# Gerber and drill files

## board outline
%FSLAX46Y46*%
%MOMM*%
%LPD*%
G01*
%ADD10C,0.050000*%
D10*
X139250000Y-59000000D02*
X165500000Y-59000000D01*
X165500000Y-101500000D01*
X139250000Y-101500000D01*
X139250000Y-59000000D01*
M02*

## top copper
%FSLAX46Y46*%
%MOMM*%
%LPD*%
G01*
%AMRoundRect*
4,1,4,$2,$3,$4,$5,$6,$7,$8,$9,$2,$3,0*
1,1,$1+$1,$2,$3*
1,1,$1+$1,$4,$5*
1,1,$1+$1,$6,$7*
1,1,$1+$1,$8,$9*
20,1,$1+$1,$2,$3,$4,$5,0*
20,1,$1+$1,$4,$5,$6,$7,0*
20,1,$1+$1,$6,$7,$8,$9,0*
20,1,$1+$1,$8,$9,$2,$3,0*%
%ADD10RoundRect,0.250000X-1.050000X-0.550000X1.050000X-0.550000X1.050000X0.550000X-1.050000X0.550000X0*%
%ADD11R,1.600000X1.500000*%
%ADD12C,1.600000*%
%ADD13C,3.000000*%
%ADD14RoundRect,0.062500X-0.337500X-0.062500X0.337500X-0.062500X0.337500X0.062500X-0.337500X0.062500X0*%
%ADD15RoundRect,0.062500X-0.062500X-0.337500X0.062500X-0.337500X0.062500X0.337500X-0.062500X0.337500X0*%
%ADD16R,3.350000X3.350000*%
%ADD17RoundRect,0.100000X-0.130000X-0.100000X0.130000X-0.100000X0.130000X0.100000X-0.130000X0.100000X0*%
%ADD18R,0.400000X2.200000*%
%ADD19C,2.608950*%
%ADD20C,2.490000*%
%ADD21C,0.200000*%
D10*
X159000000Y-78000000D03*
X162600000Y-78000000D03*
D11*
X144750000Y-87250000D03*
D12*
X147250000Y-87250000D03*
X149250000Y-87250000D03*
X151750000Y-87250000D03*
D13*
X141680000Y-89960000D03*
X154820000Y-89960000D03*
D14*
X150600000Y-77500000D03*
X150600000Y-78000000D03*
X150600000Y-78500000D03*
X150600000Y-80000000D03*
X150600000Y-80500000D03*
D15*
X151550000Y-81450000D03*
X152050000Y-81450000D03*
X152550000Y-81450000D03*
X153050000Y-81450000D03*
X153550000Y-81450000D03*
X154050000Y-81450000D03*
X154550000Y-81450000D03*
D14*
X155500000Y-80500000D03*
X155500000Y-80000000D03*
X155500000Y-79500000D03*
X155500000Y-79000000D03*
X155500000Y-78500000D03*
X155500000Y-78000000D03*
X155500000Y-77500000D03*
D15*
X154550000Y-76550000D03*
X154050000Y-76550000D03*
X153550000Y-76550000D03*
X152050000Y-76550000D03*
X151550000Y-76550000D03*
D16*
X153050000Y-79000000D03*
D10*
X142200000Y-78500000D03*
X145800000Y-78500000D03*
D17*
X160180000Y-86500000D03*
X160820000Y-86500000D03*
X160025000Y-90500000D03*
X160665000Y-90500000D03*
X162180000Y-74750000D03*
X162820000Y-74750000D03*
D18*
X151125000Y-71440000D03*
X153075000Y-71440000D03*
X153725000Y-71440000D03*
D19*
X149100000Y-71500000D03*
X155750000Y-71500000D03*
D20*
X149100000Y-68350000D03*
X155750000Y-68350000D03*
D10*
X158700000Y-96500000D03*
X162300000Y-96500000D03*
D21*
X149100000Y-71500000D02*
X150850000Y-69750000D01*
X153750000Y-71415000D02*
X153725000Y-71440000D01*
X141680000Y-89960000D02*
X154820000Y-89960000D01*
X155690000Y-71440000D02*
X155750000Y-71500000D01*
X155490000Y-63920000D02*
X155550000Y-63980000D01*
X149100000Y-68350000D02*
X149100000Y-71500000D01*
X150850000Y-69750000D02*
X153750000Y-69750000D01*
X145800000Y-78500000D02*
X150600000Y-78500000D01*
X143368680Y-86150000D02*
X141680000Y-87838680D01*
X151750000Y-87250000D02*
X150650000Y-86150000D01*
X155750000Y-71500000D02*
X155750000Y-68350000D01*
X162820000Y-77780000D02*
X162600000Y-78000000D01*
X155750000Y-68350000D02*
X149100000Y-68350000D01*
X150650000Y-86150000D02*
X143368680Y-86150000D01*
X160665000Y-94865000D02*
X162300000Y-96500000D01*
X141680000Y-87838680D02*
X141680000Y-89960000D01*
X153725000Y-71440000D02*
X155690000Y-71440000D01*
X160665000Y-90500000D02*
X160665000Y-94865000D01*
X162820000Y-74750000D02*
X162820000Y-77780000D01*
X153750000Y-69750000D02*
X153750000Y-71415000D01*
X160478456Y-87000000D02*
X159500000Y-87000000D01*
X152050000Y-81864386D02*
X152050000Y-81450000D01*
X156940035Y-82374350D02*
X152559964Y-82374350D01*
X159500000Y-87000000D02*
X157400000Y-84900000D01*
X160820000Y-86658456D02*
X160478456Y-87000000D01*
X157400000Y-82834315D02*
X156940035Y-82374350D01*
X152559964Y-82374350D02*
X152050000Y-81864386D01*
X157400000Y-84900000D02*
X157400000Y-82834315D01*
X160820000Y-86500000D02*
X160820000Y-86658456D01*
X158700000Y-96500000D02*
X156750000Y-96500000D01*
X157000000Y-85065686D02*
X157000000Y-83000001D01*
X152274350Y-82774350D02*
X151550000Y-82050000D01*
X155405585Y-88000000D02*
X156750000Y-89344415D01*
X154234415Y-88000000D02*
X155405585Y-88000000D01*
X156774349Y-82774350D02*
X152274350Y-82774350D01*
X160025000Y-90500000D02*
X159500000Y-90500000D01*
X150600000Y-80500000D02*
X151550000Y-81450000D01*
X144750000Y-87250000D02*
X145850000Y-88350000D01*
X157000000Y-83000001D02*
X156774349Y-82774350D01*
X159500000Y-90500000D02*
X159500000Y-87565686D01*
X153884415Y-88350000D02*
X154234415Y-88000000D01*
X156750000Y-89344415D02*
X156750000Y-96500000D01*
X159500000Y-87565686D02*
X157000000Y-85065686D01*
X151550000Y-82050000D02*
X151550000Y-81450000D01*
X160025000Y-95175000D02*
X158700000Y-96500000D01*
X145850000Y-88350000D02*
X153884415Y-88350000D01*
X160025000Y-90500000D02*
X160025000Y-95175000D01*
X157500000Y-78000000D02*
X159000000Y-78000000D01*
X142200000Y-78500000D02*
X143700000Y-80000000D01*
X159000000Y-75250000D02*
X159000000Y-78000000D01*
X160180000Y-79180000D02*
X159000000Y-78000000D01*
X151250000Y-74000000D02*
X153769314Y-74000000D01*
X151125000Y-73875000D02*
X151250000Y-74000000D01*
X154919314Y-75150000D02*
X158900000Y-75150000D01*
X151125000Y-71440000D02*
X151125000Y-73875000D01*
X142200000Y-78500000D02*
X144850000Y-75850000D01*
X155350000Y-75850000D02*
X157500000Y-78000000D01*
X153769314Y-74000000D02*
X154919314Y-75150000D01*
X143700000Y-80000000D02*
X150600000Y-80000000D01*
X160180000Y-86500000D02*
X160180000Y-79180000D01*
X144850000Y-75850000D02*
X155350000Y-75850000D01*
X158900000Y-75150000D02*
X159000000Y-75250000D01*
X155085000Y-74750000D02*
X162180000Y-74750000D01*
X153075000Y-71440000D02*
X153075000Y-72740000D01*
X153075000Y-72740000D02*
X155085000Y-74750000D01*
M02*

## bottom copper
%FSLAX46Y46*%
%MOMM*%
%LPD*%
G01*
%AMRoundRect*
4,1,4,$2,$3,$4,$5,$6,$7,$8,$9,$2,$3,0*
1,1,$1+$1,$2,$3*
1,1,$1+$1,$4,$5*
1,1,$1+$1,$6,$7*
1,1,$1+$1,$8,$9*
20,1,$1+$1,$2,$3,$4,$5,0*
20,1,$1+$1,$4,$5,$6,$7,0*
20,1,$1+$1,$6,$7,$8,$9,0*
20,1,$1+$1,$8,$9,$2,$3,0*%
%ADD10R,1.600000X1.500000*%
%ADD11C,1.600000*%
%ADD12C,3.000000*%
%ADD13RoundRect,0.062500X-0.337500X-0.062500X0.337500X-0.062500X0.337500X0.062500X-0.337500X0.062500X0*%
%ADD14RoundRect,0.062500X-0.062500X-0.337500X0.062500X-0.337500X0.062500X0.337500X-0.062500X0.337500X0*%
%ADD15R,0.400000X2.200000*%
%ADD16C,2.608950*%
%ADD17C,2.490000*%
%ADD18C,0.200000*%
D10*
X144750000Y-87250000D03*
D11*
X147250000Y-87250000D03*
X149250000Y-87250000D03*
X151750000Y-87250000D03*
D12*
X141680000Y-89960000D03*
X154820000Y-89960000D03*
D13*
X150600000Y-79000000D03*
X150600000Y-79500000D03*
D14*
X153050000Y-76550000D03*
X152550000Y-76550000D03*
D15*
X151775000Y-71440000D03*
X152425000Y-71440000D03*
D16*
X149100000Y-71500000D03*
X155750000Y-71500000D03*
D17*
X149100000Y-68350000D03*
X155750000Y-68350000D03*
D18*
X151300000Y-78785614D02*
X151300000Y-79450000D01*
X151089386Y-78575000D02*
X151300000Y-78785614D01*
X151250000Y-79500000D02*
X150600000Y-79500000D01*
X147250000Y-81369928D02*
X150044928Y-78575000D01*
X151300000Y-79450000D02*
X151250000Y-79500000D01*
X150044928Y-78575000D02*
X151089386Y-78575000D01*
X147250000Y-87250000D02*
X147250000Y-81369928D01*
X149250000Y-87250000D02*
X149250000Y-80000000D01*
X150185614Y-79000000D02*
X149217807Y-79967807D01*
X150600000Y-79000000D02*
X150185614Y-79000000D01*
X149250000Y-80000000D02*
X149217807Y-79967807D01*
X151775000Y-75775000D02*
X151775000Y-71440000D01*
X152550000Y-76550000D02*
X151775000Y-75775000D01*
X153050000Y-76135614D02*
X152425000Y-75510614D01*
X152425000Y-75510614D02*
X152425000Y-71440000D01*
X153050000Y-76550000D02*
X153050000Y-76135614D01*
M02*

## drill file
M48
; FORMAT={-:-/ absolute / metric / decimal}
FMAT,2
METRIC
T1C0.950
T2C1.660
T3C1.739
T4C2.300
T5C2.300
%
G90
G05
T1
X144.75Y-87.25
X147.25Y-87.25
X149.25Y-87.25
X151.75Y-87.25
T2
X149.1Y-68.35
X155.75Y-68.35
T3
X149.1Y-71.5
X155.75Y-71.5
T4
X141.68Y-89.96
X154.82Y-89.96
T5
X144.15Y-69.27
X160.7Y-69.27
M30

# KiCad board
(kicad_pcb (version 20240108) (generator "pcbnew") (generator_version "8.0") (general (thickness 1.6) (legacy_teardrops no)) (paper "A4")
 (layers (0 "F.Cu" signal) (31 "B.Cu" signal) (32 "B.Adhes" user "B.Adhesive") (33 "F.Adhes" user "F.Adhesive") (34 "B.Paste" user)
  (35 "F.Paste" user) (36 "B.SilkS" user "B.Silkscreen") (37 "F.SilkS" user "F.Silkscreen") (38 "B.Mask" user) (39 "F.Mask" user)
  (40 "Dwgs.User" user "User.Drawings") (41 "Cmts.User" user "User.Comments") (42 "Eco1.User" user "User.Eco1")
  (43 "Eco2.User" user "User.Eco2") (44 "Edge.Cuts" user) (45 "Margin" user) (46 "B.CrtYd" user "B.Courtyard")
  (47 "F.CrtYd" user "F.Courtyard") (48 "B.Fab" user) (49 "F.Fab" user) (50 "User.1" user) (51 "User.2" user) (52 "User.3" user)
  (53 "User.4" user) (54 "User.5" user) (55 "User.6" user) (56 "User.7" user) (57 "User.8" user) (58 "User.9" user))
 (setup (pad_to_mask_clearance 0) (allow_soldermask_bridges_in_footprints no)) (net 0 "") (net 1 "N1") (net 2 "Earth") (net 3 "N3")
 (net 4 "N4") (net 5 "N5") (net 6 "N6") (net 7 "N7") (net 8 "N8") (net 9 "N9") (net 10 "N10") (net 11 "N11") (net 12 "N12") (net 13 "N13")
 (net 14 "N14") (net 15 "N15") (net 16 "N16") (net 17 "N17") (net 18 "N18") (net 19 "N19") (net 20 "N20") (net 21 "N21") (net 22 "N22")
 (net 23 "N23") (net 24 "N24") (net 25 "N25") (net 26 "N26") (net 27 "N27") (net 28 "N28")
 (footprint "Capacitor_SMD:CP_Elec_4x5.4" (layer "F.Cu") (at 160.8 78)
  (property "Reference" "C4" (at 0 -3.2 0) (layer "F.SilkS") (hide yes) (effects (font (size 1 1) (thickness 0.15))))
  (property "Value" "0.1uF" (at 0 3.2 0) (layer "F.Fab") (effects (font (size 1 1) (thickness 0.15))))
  (pad "1" smd roundrect (at -1.8 0) (size 2.6 1.6) (layers "F.Cu" "F.Paste" "F.Mask") (roundrect_rratio 0.15625) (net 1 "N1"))
  (pad "2" smd roundrect (at 1.8 0) (size 2.6 1.6) (layers "F.Cu" "F.Paste" "F.Mask") (roundrect_rratio 0.15625) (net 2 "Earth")))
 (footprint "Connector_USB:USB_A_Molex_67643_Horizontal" (layer "F.Cu") (at 144.75 87.25)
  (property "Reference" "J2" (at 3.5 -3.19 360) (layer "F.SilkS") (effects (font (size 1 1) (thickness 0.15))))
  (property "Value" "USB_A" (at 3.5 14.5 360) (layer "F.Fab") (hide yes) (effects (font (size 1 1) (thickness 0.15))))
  (pad "1" thru_hole rect (at 0 0) (size 1.6 1.5) (drill 0.95) (layers "*.Cu" "*.Mask") (remove_unused_layers no) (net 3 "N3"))
  (pad "2" thru_hole circle (at 2.5 0) (size 1.6 1.6) (drill 0.95) (layers "*.Cu" "*.Mask") (remove_unused_layers no) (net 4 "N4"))
  (pad "3" thru_hole circle (at 4.5 0) (size 1.6 1.6) (drill 0.95) (layers "*.Cu" "*.Mask") (remove_unused_layers no) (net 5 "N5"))
  (pad "4" thru_hole circle (at 7 0) (size 1.6 1.6) (drill 0.95) (layers "*.Cu" "*.Mask") (remove_unused_layers no) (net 2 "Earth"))
  (pad "5" thru_hole circle (at -3.07 2.71) (size 3 3) (drill 2.3) (layers "*.Cu" "*.Mask") (remove_unused_layers no) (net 2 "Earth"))
  (pad "5" thru_hole circle (at 10.07 2.71) (size 3 3) (drill 2.3) (layers "*.Cu" "*.Mask") (remove_unused_layers no) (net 2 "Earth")))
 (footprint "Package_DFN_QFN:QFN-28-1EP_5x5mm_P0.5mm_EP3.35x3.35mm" (layer "F.Cu") (at 153.05 79)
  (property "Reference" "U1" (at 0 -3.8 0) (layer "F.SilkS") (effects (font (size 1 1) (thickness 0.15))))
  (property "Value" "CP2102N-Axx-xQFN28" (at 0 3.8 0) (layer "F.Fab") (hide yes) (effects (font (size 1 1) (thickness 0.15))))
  (pad "" smd roundrect (at -1.12 -1.12) (size 0.9 0.9) (layers "F.Paste") (roundrect_rratio 0.25))
  (pad "" smd roundrect (at -1.12 0) (size 0.9 0.9) (layers "F.Paste") (roundrect_rratio 0.25))
  (pad "" smd roundrect (at -1.12 1.12) (size 0.9 0.9) (layers "F.Paste") (roundrect_rratio 0.25))
  (pad "" smd roundrect (at 0 -1.12) (size 0.9 0.9) (layers "F.Paste") (roundrect_rratio 0.25))
  (pad "" smd roundrect (at 0 0) (size 0.9 0.9) (layers "F.Paste") (roundrect_rratio 0.25))
  (pad "" smd roundrect (at 0 1.12) (size 0.9 0.9) (layers "F.Paste") (roundrect_rratio 0.25))
  (pad "" smd roundrect (at 1.12 -1.12) (size 0.9 0.9) (layers "F.Paste") (roundrect_rratio 0.25))
  (pad "" smd roundrect (at 1.12 0) (size 0.9 0.9) (layers "F.Paste") (roundrect_rratio 0.25))
  (pad "" smd roundrect (at 1.12 1.12) (size 0.9 0.9) (layers "F.Paste") (roundrect_rratio 0.25))
  (pad "1" smd roundrect (at -2.45 -1.5) (size 0.8 0.25) (layers "F.Cu" "F.Paste" "F.Mask") (roundrect_rratio 0.25) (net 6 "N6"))
  (pad "2" smd roundrect (at -2.45 -1) (size 0.8 0.25) (layers "F.Cu" "F.Paste" "F.Mask") (roundrect_rratio 0.25) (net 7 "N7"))
  (pad "3" smd roundrect (at -2.45 -0.5) (size 0.8 0.25) (layers "F.Cu" "F.Paste" "F.Mask") (roundrect_rratio 0.25) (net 2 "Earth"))
  (pad "4" smd roundrect (at -2.45 0) (size 0.8 0.25) (layers "B.Cu" "F.Paste" "F.Mask") (roundrect_rratio 0.25) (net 5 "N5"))
  (pad "5" smd roundrect (at -2.45 0.5) (size 0.8 0.25) (layers "B.Cu" "F.Paste" "F.Mask") (roundrect_rratio 0.25) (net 4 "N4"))
  (pad "6" smd roundrect (at -2.45 1) (size 0.8 0.25) (layers "F.Cu" "F.Paste" "F.Mask") (roundrect_rratio 0.25) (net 1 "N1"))
  (pad "7" smd roundrect (at -2.45 1.5) (size 0.8 0.25) (layers "F.Cu" "F.Paste" "F.Mask") (roundrect_rratio 0.25) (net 3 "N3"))
  (pad "8" smd roundrect (at -1.5 2.45) (size 0.25 0.8) (layers "F.Cu" "F.Paste" "F.Mask") (roundrect_rratio 0.25) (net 3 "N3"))
  (pad "9" smd roundrect (at -1 2.45) (size 0.25 0.8) (layers "F.Cu" "F.Paste" "F.Mask") (roundrect_rratio 0.25) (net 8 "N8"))
  (pad "10" smd roundrect (at -0.5 2.45) (size 0.25 0.8) (layers "F.Cu" "F.Paste" "F.Mask") (roundrect_rratio 0.25) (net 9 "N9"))
  (pad "11" smd roundrect (at 0 2.45) (size 0.25 0.8) (layers "F.Cu" "F.Paste" "F.Mask") (roundrect_rratio 0.25) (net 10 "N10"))
  (pad "12" smd roundrect (at 0.5 2.45) (size 0.25 0.8) (layers "F.Cu" "F.Paste" "F.Mask") (roundrect_rratio 0.25) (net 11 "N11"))
  (pad "13" smd roundrect (at 1 2.45) (size 0.25 0.8) (layers "F.Cu" "F.Paste" "F.Mask") (roundrect_rratio 0.25) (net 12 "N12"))
  (pad "14" smd roundrect (at 1.5 2.45) (size 0.25 0.8) (layers "F.Cu" "F.Paste" "F.Mask") (roundrect_rratio 0.25) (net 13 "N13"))
  (pad "15" smd roundrect (at 2.45 1.5) (size 0.8 0.25) (layers "F.Cu" "F.Paste" "F.Mask") (roundrect_rratio 0.25) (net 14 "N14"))
  (pad "16" smd roundrect (at 2.45 1) (size 0.8 0.25) (layers "F.Cu" "F.Paste" "F.Mask") (roundrect_rratio 0.25) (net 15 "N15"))
  (pad "17" smd roundrect (at 2.45 0.5) (size 0.8 0.25) (layers "F.Cu" "F.Paste" "F.Mask") (roundrect_rratio 0.25) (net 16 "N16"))
  (pad "18" smd roundrect (at 2.45 0) (size 0.8 0.25) (layers "F.Cu" "F.Paste" "F.Mask") (roundrect_rratio 0.25) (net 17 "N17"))
  (pad "19" smd roundrect (at 2.45 -0.5) (size 0.8 0.25) (layers "F.Cu" "F.Paste" "F.Mask") (roundrect_rratio 0.25) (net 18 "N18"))
  (pad "20" smd roundrect (at 2.45 -1) (size 0.8 0.25) (layers "F.Cu" "F.Paste" "F.Mask") (roundrect_rratio 0.25) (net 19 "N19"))
  (pad "21" smd roundrect (at 2.45 -1.5) (size 0.8 0.25) (layers "F.Cu" "F.Paste" "F.Mask") (roundrect_rratio 0.25) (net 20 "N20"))
  (pad "22" smd roundrect (at 1.5 -2.45) (size 0.25 0.8) (layers "F.Cu" "F.Paste" "F.Mask") (roundrect_rratio 0.25) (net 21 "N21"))
  (pad "23" smd roundrect (at 1 -2.45) (size 0.25 0.8) (layers "F.Cu" "F.Paste" "F.Mask") (roundrect_rratio 0.25) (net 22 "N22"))
  (pad "24" smd roundrect (at 0.5 -2.45) (size 0.25 0.8) (layers "F.Cu" "F.Paste" "F.Mask") (roundrect_rratio 0.25) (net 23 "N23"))
  (pad "25" smd roundrect (at 0 -2.45) (size 0.25 0.8) (layers "B.Cu" "F.Paste" "F.Mask") (roundrect_rratio 0.25) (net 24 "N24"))
  (pad "26" smd roundrect (at -0.5 -2.45) (size 0.25 0.8) (layers "B.Cu" "F.Paste" "F.Mask") (roundrect_rratio 0.25) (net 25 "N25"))
  (pad "27" smd roundrect (at -1 -2.45) (size 0.25 0.8) (layers "F.Cu" "F.Paste" "F.Mask") (roundrect_rratio 0.25) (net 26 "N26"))
  (pad "28" smd roundrect (at -1.5 -2.45) (size 0.25 0.8) (layers "F.Cu" "F.Paste" "F.Mask") (roundrect_rratio 0.25) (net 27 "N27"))
  (pad "29" smd rect (at 0 0) (size 3.35 3.35) (layers "F.Cu" "F.Mask") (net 2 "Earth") (zone_connect 2)))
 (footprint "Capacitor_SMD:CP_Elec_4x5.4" (layer "F.Cu") (at 144 78.5)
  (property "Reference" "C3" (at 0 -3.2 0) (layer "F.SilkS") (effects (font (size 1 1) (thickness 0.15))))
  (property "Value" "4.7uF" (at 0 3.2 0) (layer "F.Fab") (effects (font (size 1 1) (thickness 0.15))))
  (pad "1" smd roundrect (at -1.8 0) (size 2.6 1.6) (layers "F.Cu" "F.Paste" "F.Mask") (roundrect_rratio 0.15625) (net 1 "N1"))
  (pad "2" smd roundrect (at 1.8 0) (size 2.6 1.6) (layers "F.Cu" "F.Paste" "F.Mask") (roundrect_rratio 0.15625) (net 2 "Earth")))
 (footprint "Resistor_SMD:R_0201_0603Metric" (layer "F.Cu") (at 160.5 86.5)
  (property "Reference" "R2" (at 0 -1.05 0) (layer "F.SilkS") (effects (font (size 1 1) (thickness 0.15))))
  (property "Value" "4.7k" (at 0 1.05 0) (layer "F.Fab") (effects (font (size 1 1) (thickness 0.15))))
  (pad "" smd roundrect (at -0.345 0) (size 0.318 0.36) (layers "F.Paste") (roundrect_rratio 0.25))
  (pad "" smd roundrect (at 0.345 0) (size 0.318 0.36) (layers "F.Paste") (roundrect_rratio 0.25))
  (pad "1" smd roundrect (at -0.32 0) (size 0.46 0.4) (layers "F.Cu" "F.Mask") (roundrect_rratio 0.25) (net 1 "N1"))
  (pad "2" smd roundrect (at 0.32 0) (size 0.46 0.4) (layers "F.Cu" "F.Mask") (roundrect_rratio 0.25) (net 8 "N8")))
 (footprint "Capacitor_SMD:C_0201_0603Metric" (layer "F.Cu") (at 160.345 90.5)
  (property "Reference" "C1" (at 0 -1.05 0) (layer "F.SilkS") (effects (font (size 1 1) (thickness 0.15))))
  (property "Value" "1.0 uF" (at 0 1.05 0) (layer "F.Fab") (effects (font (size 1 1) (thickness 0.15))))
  (pad "" smd roundrect (at -0.345 0) (size 0.318 0.36) (layers "F.Paste") (roundrect_rratio 0.25))
  (pad "" smd roundrect (at 0.345 0) (size 0.318 0.36) (layers "F.Paste") (roundrect_rratio 0.25))
  (pad "1" smd roundrect (at -0.32 0) (size 0.46 0.4) (layers "F.Cu" "F.Mask") (roundrect_rratio 0.25) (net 3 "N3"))
  (pad "2" smd roundrect (at 0.32 0) (size 0.46 0.4) (layers "F.Cu" "F.Mask") (roundrect_rratio 0.25) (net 2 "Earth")))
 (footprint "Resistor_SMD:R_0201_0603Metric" (layer "F.Cu") (at 162.5 74.75)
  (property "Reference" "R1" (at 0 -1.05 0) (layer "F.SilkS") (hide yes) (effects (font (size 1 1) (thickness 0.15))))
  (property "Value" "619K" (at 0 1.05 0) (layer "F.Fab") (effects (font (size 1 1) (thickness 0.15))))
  (pad "" smd roundrect (at -0.345 0) (size 0.318 0.36) (layers "F.Paste") (roundrect_rratio 0.25))
  (pad "" smd roundrect (at 0.345 0) (size 0.318 0.36) (layers "F.Paste") (roundrect_rratio 0.25))
  (pad "1" smd roundrect (at -0.32 0) (size 0.46 0.4) (layers "F.Cu" "F.Mask") (roundrect_rratio 0.25) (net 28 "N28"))
  (pad "2" smd roundrect (at 0.32 0) (size 0.46 0.4) (layers "F.Cu" "F.Mask") (roundrect_rratio 0.25) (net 2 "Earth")))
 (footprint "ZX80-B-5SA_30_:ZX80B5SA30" (layer "F.Cu") (at 152.425 69.462)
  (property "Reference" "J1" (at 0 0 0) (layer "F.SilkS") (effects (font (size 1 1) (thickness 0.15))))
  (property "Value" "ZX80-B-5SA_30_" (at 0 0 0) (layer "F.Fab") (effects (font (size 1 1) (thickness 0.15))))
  (pad "" np_thru_hole circle (at -8.275 -0.192) (size 2.3 2.3) (drill 2.3) (layers "*.Cu" "*.Mask"))
  (pad "" np_thru_hole circle (at 8.275 -0.192) (size 2.3 2.3) (drill 2.3) (layers "*.Cu" "*.Mask"))
  (pad "1" smd rect (at -1.3 1.978 90) (size 2.2 0.4) (layers "F.Cu" "F.Paste" "F.Mask") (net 1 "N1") (solder_mask_margin 0.102))
  (pad "2" smd rect (at -0.65 1.978 90) (size 2.2 0.4) (layers "B.Cu" "F.Paste" "F.Mask") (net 25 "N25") (solder_mask_margin 0.102))
  (pad "3" smd rect (at 0 1.978 90) (size 2.2 0.4) (layers "B.Cu" "F.Paste" "F.Mask") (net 24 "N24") (solder_mask_margin 0.102))
  (pad "4" smd rect (at 0.65 1.978 90) (size 2.2 0.4) (layers "F.Cu" "F.Paste" "F.Mask") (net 28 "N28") (solder_mask_margin 0.102))
  (pad "5" smd rect (at 1.3 1.978 90) (size 2.2 0.4) (layers "F.Cu" "F.Paste" "F.Mask") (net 2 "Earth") (solder_mask_margin 0.102))
  (pad "6" thru_hole circle (at -3.325 2.038) (size 2.60895 2.60895) (drill 1.7393) (layers "*.Cu" "*.Mask") (remove_unused_layers no)
   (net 2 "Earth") (solder_mask_margin 0.102))
  (pad "7" thru_hole circle (at 3.325 2.038) (size 2.60895 2.60895) (drill 1.7393) (layers "*.Cu" "*.Mask") (remove_unused_layers no)
   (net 2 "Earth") (solder_mask_margin 0.102))
  (pad "8" thru_hole circle (at -3.325 -1.112) (size 2.49 2.49) (drill 1.66) (layers "*.Cu" "*.Mask") (remove_unused_layers no)
   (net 2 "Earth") (solder_mask_margin 0.102))
  (pad "9" thru_hole circle (at 3.325 -1.112) (size 2.49 2.49) (drill 1.66) (layers "*.Cu" "*.Mask") (remove_unused_layers no)
   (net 2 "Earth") (solder_mask_margin 0.102)))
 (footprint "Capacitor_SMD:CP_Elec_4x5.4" (layer "F.Cu") (at 160.5 96.5)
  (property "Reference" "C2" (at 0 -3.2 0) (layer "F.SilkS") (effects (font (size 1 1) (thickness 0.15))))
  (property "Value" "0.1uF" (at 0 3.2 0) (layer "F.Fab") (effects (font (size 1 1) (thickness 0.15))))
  (pad "1" smd roundrect (at -1.8 0) (size 2.6 1.6) (layers "F.Cu" "F.Paste" "F.Mask") (roundrect_rratio 0.15625) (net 3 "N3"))
  (pad "2" smd roundrect (at 1.8 0) (size 2.6 1.6) (layers "F.Cu" "F.Paste" "F.Mask") (roundrect_rratio 0.15625) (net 2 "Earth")))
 (gr_rect (start 139.25 59) (end 165.5 101.5) (stroke (width 0.05) (type default)) (fill none) (layer "Edge.Cuts"))
 (segment (start 149.1 71.5) (end 150.85 69.75) (width 0.2) (layer "F.Cu") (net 2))
 (segment (start 153.75 71.415) (end 153.725 71.44) (width 0.2) (layer "F.Cu") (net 2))
 (segment (start 141.68 89.96) (end 154.82 89.96) (width 0.2) (layer "F.Cu") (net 2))
 (segment (start 155.69 71.44) (end 155.75 71.5) (width 0.2) (layer "F.Cu") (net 2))
 (segment (start 155.49 63.92) (end 155.55 63.98) (width 0.2) (layer "F.Cu") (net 2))
 (segment (start 149.1 68.35) (end 149.1 71.5) (width 0.2) (layer "F.Cu") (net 2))
 (segment (start 150.85 69.75) (end 153.75 69.75) (width 0.2) (layer "F.Cu") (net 2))
 (segment (start 145.8 78.5) (end 150.6 78.5) (width 0.2) (layer "F.Cu") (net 2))
 (segment (start 143.36868 86.15) (end 141.68 87.83868) (width 0.2) (layer "F.Cu") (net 2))
 (segment (start 151.75 87.25) (end 150.65 86.15) (width 0.2) (layer "F.Cu") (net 2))
 (segment (start 155.75 71.5) (end 155.75 68.35) (width 0.2) (layer "F.Cu") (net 2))
 (segment (start 162.82 77.78) (end 162.6 78) (width 0.2) (layer "F.Cu") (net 2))
 (segment (start 155.75 68.35) (end 149.1 68.35) (width 0.2) (layer "F.Cu") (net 2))
 (segment (start 150.65 86.15) (end 143.36868 86.15) (width 0.2) (layer "F.Cu") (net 2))
 (segment (start 160.665 94.865) (end 162.3 96.5) (width 0.2) (layer "F.Cu") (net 2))
 (segment (start 141.68 87.83868) (end 141.68 89.96) (width 0.2) (layer "F.Cu") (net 2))
 (segment (start 153.725 71.44) (end 155.69 71.44) (width 0.2) (layer "F.Cu") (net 2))
 (segment (start 160.665 90.5) (end 160.665 94.865) (width 0.2) (layer "F.Cu") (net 2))
 (segment (start 162.82 74.75) (end 162.82 77.78) (width 0.2) (layer "F.Cu") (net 2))
 (segment (start 153.75 69.75) (end 153.75 71.415) (width 0.2) (layer "F.Cu") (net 2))
 (segment (start 151.3 78.785614) (end 151.3 79.45) (width 0.2) (layer "B.Cu") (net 4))
 (segment (start 151.089386 78.575) (end 151.3 78.785614) (width 0.2) (layer "B.Cu") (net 4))
 (segment (start 151.25 79.5) (end 150.6 79.5) (width 0.2) (layer "B.Cu") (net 4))
 (segment (start 147.25 81.369928) (end 150.044928 78.575) (width 0.2) (layer "B.Cu") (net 4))
 (segment (start 151.3 79.45) (end 151.25 79.5) (width 0.2) (layer "B.Cu") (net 4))
 (segment (start 150.044928 78.575) (end 151.089386 78.575) (width 0.2) (layer "B.Cu") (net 4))
 (segment (start 147.25 87.25) (end 147.25 81.369928) (width 0.2) (layer "B.Cu") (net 4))
 (segment (start 149.25 87.25) (end 149.25 80) (width 0.2) (layer "B.Cu") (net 5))
 (segment (start 150.185614 79) (end 149.217807 79.967807) (width 0.2) (layer "B.Cu") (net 5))
 (segment (start 150.6 79) (end 150.185614 79) (width 0.2) (layer "B.Cu") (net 5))
 (segment (start 149.25 80) (end 149.217807 79.967807) (width 0.2) (layer "B.Cu") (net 5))
 (segment (start 160.478456 87) (end 159.5 87) (width 0.2) (layer "F.Cu") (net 8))
 (segment (start 152.05 81.864386) (end 152.05 81.45) (width 0.2) (layer "F.Cu") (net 8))
 (segment (start 156.940035 82.37435) (end 152.559964 82.37435) (width 0.2) (layer "F.Cu") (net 8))
 (segment (start 159.5 87) (end 157.4 84.9) (width 0.2) (layer "F.Cu") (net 8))
 (segment (start 160.82 86.658456) (end 160.478456 87) (width 0.2) (layer "F.Cu") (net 8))
 (segment (start 157.4 82.834315) (end 156.940035 82.37435) (width 0.2) (layer "F.Cu") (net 8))
 (segment (start 152.559964 82.37435) (end 152.05 81.864386) (width 0.2) (layer "F.Cu") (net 8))
 (segment (start 157.4 84.9) (end 157.4 82.834315) (width 0.2) (layer "F.Cu") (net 8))
 (segment (start 160.82 86.5) (end 160.82 86.658456) (width 0.2) (layer "F.Cu") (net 8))
 (segment (start 158.7 96.5) (end 156.75 96.5) (width 0.2) (layer "F.Cu") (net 3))
 (segment (start 157 85.065686) (end 157 83.000001) (width 0.2) (layer "F.Cu") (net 3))
 (segment (start 152.27435 82.77435) (end 151.55 82.05) (width 0.2) (layer "F.Cu") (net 3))
 (segment (start 155.405585 88) (end 156.75 89.344415) (width 0.2) (layer "F.Cu") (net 3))
 (segment (start 154.234415 88) (end 155.405585 88) (width 0.2) (layer "F.Cu") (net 3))
 (segment (start 156.774349 82.77435) (end 152.27435 82.77435) (width 0.2) (layer "F.Cu") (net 3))
 (segment (start 160.025 90.5) (end 159.5 90.5) (width 0.2) (layer "F.Cu") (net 3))
 (segment (start 150.6 80.5) (end 151.55 81.45) (width 0.2) (layer "F.Cu") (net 3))
 (segment (start 144.75 87.25) (end 145.85 88.35) (width 0.2) (layer "F.Cu") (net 3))
 (segment (start 157 83.000001) (end 156.774349 82.77435) (width 0.2) (layer "F.Cu") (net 3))
 (segment (start 159.5 90.5) (end 159.5 87.565686) (width 0.2) (layer "F.Cu") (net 3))
 (segment (start 153.884415 88.35) (end 154.234415 88) (width 0.2) (layer "F.Cu") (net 3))
 (segment (start 156.75 89.344415) (end 156.75 96.5) (width 0.2) (layer "F.Cu") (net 3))
 (segment (start 159.5 87.565686) (end 157 85.065686) (width 0.2) (layer "F.Cu") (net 3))
 (segment (start 151.55 82.05) (end 151.55 81.45) (width 0.2) (layer "F.Cu") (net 3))
 (segment (start 160.025 95.175) (end 158.7 96.5) (width 0.2) (layer "F.Cu") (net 3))
 (segment (start 145.85 88.35) (end 153.884415 88.35) (width 0.2) (layer "F.Cu") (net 3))
 (segment (start 160.025 90.5) (end 160.025 95.175) (width 0.2) (layer "F.Cu") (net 3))
 (segment (start 157.5 78) (end 159 78) (width 0.2) (layer "F.Cu") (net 1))
 (segment (start 142.2 78.5) (end 143.7 80) (width 0.2) (layer "F.Cu") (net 1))
 (segment (start 159 75.25) (end 159 78) (width 0.2) (layer "F.Cu") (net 1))
 (segment (start 160.18 79.18) (end 159 78) (width 0.2) (layer "F.Cu") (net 1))
 (segment (start 151.25 74) (end 153.769314 74) (width 0.2) (layer "F.Cu") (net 1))
 (segment (start 151.125 73.875) (end 151.25 74) (width 0.2) (layer "F.Cu") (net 1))
 (segment (start 154.919314 75.15) (end 158.9 75.15) (width 0.2) (layer "F.Cu") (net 1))
 (segment (start 151.125 71.44) (end 151.125 73.875) (width 0.2) (layer "F.Cu") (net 1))
 (segment (start 142.2 78.5) (end 144.85 75.85) (width 0.2) (layer "F.Cu") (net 1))
 (segment (start 155.35 75.85) (end 157.5 78) (width 0.2) (layer "F.Cu") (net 1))
 (segment (start 153.769314 74) (end 154.919314 75.15) (width 0.2) (layer "F.Cu") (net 1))
 (segment (start 143.7 80) (end 150.6 80) (width 0.2) (layer "F.Cu") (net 1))
 (segment (start 160.18 86.5) (end 160.18 79.18) (width 0.2) (layer "F.Cu") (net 1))
 (segment (start 144.85 75.85) (end 155.35 75.85) (width 0.2) (layer "F.Cu") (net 1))
 (segment (start 158.9 75.15) (end 159 75.25) (width 0.2) (layer "F.Cu") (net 1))
 (segment (start 151.775 75.775) (end 151.775 71.44) (width 0.2) (layer "B.Cu") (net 25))
 (segment (start 152.55 76.55) (end 151.775 75.775) (width 0.2) (layer "B.Cu") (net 25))
 (segment (start 155.085 74.75) (end 162.18 74.75) (width 0.2) (layer "F.Cu") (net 28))
 (segment (start 153.075 71.44) (end 153.075 72.74) (width 0.2) (layer "F.Cu") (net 28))
 (segment (start 153.075 72.74) (end 155.085 74.75) (width 0.2) (layer "F.Cu") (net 28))
 (segment (start 153.05 76.135614) (end 152.425 75.510614) (width 0.2) (layer "B.Cu") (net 24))
 (segment (start 152.425 75.510614) (end 152.425 71.44) (width 0.2) (layer "B.Cu") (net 24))
 (segment (start 153.05 76.55) (end 153.05 76.135614) (width 0.2) (layer "B.Cu") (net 24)))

